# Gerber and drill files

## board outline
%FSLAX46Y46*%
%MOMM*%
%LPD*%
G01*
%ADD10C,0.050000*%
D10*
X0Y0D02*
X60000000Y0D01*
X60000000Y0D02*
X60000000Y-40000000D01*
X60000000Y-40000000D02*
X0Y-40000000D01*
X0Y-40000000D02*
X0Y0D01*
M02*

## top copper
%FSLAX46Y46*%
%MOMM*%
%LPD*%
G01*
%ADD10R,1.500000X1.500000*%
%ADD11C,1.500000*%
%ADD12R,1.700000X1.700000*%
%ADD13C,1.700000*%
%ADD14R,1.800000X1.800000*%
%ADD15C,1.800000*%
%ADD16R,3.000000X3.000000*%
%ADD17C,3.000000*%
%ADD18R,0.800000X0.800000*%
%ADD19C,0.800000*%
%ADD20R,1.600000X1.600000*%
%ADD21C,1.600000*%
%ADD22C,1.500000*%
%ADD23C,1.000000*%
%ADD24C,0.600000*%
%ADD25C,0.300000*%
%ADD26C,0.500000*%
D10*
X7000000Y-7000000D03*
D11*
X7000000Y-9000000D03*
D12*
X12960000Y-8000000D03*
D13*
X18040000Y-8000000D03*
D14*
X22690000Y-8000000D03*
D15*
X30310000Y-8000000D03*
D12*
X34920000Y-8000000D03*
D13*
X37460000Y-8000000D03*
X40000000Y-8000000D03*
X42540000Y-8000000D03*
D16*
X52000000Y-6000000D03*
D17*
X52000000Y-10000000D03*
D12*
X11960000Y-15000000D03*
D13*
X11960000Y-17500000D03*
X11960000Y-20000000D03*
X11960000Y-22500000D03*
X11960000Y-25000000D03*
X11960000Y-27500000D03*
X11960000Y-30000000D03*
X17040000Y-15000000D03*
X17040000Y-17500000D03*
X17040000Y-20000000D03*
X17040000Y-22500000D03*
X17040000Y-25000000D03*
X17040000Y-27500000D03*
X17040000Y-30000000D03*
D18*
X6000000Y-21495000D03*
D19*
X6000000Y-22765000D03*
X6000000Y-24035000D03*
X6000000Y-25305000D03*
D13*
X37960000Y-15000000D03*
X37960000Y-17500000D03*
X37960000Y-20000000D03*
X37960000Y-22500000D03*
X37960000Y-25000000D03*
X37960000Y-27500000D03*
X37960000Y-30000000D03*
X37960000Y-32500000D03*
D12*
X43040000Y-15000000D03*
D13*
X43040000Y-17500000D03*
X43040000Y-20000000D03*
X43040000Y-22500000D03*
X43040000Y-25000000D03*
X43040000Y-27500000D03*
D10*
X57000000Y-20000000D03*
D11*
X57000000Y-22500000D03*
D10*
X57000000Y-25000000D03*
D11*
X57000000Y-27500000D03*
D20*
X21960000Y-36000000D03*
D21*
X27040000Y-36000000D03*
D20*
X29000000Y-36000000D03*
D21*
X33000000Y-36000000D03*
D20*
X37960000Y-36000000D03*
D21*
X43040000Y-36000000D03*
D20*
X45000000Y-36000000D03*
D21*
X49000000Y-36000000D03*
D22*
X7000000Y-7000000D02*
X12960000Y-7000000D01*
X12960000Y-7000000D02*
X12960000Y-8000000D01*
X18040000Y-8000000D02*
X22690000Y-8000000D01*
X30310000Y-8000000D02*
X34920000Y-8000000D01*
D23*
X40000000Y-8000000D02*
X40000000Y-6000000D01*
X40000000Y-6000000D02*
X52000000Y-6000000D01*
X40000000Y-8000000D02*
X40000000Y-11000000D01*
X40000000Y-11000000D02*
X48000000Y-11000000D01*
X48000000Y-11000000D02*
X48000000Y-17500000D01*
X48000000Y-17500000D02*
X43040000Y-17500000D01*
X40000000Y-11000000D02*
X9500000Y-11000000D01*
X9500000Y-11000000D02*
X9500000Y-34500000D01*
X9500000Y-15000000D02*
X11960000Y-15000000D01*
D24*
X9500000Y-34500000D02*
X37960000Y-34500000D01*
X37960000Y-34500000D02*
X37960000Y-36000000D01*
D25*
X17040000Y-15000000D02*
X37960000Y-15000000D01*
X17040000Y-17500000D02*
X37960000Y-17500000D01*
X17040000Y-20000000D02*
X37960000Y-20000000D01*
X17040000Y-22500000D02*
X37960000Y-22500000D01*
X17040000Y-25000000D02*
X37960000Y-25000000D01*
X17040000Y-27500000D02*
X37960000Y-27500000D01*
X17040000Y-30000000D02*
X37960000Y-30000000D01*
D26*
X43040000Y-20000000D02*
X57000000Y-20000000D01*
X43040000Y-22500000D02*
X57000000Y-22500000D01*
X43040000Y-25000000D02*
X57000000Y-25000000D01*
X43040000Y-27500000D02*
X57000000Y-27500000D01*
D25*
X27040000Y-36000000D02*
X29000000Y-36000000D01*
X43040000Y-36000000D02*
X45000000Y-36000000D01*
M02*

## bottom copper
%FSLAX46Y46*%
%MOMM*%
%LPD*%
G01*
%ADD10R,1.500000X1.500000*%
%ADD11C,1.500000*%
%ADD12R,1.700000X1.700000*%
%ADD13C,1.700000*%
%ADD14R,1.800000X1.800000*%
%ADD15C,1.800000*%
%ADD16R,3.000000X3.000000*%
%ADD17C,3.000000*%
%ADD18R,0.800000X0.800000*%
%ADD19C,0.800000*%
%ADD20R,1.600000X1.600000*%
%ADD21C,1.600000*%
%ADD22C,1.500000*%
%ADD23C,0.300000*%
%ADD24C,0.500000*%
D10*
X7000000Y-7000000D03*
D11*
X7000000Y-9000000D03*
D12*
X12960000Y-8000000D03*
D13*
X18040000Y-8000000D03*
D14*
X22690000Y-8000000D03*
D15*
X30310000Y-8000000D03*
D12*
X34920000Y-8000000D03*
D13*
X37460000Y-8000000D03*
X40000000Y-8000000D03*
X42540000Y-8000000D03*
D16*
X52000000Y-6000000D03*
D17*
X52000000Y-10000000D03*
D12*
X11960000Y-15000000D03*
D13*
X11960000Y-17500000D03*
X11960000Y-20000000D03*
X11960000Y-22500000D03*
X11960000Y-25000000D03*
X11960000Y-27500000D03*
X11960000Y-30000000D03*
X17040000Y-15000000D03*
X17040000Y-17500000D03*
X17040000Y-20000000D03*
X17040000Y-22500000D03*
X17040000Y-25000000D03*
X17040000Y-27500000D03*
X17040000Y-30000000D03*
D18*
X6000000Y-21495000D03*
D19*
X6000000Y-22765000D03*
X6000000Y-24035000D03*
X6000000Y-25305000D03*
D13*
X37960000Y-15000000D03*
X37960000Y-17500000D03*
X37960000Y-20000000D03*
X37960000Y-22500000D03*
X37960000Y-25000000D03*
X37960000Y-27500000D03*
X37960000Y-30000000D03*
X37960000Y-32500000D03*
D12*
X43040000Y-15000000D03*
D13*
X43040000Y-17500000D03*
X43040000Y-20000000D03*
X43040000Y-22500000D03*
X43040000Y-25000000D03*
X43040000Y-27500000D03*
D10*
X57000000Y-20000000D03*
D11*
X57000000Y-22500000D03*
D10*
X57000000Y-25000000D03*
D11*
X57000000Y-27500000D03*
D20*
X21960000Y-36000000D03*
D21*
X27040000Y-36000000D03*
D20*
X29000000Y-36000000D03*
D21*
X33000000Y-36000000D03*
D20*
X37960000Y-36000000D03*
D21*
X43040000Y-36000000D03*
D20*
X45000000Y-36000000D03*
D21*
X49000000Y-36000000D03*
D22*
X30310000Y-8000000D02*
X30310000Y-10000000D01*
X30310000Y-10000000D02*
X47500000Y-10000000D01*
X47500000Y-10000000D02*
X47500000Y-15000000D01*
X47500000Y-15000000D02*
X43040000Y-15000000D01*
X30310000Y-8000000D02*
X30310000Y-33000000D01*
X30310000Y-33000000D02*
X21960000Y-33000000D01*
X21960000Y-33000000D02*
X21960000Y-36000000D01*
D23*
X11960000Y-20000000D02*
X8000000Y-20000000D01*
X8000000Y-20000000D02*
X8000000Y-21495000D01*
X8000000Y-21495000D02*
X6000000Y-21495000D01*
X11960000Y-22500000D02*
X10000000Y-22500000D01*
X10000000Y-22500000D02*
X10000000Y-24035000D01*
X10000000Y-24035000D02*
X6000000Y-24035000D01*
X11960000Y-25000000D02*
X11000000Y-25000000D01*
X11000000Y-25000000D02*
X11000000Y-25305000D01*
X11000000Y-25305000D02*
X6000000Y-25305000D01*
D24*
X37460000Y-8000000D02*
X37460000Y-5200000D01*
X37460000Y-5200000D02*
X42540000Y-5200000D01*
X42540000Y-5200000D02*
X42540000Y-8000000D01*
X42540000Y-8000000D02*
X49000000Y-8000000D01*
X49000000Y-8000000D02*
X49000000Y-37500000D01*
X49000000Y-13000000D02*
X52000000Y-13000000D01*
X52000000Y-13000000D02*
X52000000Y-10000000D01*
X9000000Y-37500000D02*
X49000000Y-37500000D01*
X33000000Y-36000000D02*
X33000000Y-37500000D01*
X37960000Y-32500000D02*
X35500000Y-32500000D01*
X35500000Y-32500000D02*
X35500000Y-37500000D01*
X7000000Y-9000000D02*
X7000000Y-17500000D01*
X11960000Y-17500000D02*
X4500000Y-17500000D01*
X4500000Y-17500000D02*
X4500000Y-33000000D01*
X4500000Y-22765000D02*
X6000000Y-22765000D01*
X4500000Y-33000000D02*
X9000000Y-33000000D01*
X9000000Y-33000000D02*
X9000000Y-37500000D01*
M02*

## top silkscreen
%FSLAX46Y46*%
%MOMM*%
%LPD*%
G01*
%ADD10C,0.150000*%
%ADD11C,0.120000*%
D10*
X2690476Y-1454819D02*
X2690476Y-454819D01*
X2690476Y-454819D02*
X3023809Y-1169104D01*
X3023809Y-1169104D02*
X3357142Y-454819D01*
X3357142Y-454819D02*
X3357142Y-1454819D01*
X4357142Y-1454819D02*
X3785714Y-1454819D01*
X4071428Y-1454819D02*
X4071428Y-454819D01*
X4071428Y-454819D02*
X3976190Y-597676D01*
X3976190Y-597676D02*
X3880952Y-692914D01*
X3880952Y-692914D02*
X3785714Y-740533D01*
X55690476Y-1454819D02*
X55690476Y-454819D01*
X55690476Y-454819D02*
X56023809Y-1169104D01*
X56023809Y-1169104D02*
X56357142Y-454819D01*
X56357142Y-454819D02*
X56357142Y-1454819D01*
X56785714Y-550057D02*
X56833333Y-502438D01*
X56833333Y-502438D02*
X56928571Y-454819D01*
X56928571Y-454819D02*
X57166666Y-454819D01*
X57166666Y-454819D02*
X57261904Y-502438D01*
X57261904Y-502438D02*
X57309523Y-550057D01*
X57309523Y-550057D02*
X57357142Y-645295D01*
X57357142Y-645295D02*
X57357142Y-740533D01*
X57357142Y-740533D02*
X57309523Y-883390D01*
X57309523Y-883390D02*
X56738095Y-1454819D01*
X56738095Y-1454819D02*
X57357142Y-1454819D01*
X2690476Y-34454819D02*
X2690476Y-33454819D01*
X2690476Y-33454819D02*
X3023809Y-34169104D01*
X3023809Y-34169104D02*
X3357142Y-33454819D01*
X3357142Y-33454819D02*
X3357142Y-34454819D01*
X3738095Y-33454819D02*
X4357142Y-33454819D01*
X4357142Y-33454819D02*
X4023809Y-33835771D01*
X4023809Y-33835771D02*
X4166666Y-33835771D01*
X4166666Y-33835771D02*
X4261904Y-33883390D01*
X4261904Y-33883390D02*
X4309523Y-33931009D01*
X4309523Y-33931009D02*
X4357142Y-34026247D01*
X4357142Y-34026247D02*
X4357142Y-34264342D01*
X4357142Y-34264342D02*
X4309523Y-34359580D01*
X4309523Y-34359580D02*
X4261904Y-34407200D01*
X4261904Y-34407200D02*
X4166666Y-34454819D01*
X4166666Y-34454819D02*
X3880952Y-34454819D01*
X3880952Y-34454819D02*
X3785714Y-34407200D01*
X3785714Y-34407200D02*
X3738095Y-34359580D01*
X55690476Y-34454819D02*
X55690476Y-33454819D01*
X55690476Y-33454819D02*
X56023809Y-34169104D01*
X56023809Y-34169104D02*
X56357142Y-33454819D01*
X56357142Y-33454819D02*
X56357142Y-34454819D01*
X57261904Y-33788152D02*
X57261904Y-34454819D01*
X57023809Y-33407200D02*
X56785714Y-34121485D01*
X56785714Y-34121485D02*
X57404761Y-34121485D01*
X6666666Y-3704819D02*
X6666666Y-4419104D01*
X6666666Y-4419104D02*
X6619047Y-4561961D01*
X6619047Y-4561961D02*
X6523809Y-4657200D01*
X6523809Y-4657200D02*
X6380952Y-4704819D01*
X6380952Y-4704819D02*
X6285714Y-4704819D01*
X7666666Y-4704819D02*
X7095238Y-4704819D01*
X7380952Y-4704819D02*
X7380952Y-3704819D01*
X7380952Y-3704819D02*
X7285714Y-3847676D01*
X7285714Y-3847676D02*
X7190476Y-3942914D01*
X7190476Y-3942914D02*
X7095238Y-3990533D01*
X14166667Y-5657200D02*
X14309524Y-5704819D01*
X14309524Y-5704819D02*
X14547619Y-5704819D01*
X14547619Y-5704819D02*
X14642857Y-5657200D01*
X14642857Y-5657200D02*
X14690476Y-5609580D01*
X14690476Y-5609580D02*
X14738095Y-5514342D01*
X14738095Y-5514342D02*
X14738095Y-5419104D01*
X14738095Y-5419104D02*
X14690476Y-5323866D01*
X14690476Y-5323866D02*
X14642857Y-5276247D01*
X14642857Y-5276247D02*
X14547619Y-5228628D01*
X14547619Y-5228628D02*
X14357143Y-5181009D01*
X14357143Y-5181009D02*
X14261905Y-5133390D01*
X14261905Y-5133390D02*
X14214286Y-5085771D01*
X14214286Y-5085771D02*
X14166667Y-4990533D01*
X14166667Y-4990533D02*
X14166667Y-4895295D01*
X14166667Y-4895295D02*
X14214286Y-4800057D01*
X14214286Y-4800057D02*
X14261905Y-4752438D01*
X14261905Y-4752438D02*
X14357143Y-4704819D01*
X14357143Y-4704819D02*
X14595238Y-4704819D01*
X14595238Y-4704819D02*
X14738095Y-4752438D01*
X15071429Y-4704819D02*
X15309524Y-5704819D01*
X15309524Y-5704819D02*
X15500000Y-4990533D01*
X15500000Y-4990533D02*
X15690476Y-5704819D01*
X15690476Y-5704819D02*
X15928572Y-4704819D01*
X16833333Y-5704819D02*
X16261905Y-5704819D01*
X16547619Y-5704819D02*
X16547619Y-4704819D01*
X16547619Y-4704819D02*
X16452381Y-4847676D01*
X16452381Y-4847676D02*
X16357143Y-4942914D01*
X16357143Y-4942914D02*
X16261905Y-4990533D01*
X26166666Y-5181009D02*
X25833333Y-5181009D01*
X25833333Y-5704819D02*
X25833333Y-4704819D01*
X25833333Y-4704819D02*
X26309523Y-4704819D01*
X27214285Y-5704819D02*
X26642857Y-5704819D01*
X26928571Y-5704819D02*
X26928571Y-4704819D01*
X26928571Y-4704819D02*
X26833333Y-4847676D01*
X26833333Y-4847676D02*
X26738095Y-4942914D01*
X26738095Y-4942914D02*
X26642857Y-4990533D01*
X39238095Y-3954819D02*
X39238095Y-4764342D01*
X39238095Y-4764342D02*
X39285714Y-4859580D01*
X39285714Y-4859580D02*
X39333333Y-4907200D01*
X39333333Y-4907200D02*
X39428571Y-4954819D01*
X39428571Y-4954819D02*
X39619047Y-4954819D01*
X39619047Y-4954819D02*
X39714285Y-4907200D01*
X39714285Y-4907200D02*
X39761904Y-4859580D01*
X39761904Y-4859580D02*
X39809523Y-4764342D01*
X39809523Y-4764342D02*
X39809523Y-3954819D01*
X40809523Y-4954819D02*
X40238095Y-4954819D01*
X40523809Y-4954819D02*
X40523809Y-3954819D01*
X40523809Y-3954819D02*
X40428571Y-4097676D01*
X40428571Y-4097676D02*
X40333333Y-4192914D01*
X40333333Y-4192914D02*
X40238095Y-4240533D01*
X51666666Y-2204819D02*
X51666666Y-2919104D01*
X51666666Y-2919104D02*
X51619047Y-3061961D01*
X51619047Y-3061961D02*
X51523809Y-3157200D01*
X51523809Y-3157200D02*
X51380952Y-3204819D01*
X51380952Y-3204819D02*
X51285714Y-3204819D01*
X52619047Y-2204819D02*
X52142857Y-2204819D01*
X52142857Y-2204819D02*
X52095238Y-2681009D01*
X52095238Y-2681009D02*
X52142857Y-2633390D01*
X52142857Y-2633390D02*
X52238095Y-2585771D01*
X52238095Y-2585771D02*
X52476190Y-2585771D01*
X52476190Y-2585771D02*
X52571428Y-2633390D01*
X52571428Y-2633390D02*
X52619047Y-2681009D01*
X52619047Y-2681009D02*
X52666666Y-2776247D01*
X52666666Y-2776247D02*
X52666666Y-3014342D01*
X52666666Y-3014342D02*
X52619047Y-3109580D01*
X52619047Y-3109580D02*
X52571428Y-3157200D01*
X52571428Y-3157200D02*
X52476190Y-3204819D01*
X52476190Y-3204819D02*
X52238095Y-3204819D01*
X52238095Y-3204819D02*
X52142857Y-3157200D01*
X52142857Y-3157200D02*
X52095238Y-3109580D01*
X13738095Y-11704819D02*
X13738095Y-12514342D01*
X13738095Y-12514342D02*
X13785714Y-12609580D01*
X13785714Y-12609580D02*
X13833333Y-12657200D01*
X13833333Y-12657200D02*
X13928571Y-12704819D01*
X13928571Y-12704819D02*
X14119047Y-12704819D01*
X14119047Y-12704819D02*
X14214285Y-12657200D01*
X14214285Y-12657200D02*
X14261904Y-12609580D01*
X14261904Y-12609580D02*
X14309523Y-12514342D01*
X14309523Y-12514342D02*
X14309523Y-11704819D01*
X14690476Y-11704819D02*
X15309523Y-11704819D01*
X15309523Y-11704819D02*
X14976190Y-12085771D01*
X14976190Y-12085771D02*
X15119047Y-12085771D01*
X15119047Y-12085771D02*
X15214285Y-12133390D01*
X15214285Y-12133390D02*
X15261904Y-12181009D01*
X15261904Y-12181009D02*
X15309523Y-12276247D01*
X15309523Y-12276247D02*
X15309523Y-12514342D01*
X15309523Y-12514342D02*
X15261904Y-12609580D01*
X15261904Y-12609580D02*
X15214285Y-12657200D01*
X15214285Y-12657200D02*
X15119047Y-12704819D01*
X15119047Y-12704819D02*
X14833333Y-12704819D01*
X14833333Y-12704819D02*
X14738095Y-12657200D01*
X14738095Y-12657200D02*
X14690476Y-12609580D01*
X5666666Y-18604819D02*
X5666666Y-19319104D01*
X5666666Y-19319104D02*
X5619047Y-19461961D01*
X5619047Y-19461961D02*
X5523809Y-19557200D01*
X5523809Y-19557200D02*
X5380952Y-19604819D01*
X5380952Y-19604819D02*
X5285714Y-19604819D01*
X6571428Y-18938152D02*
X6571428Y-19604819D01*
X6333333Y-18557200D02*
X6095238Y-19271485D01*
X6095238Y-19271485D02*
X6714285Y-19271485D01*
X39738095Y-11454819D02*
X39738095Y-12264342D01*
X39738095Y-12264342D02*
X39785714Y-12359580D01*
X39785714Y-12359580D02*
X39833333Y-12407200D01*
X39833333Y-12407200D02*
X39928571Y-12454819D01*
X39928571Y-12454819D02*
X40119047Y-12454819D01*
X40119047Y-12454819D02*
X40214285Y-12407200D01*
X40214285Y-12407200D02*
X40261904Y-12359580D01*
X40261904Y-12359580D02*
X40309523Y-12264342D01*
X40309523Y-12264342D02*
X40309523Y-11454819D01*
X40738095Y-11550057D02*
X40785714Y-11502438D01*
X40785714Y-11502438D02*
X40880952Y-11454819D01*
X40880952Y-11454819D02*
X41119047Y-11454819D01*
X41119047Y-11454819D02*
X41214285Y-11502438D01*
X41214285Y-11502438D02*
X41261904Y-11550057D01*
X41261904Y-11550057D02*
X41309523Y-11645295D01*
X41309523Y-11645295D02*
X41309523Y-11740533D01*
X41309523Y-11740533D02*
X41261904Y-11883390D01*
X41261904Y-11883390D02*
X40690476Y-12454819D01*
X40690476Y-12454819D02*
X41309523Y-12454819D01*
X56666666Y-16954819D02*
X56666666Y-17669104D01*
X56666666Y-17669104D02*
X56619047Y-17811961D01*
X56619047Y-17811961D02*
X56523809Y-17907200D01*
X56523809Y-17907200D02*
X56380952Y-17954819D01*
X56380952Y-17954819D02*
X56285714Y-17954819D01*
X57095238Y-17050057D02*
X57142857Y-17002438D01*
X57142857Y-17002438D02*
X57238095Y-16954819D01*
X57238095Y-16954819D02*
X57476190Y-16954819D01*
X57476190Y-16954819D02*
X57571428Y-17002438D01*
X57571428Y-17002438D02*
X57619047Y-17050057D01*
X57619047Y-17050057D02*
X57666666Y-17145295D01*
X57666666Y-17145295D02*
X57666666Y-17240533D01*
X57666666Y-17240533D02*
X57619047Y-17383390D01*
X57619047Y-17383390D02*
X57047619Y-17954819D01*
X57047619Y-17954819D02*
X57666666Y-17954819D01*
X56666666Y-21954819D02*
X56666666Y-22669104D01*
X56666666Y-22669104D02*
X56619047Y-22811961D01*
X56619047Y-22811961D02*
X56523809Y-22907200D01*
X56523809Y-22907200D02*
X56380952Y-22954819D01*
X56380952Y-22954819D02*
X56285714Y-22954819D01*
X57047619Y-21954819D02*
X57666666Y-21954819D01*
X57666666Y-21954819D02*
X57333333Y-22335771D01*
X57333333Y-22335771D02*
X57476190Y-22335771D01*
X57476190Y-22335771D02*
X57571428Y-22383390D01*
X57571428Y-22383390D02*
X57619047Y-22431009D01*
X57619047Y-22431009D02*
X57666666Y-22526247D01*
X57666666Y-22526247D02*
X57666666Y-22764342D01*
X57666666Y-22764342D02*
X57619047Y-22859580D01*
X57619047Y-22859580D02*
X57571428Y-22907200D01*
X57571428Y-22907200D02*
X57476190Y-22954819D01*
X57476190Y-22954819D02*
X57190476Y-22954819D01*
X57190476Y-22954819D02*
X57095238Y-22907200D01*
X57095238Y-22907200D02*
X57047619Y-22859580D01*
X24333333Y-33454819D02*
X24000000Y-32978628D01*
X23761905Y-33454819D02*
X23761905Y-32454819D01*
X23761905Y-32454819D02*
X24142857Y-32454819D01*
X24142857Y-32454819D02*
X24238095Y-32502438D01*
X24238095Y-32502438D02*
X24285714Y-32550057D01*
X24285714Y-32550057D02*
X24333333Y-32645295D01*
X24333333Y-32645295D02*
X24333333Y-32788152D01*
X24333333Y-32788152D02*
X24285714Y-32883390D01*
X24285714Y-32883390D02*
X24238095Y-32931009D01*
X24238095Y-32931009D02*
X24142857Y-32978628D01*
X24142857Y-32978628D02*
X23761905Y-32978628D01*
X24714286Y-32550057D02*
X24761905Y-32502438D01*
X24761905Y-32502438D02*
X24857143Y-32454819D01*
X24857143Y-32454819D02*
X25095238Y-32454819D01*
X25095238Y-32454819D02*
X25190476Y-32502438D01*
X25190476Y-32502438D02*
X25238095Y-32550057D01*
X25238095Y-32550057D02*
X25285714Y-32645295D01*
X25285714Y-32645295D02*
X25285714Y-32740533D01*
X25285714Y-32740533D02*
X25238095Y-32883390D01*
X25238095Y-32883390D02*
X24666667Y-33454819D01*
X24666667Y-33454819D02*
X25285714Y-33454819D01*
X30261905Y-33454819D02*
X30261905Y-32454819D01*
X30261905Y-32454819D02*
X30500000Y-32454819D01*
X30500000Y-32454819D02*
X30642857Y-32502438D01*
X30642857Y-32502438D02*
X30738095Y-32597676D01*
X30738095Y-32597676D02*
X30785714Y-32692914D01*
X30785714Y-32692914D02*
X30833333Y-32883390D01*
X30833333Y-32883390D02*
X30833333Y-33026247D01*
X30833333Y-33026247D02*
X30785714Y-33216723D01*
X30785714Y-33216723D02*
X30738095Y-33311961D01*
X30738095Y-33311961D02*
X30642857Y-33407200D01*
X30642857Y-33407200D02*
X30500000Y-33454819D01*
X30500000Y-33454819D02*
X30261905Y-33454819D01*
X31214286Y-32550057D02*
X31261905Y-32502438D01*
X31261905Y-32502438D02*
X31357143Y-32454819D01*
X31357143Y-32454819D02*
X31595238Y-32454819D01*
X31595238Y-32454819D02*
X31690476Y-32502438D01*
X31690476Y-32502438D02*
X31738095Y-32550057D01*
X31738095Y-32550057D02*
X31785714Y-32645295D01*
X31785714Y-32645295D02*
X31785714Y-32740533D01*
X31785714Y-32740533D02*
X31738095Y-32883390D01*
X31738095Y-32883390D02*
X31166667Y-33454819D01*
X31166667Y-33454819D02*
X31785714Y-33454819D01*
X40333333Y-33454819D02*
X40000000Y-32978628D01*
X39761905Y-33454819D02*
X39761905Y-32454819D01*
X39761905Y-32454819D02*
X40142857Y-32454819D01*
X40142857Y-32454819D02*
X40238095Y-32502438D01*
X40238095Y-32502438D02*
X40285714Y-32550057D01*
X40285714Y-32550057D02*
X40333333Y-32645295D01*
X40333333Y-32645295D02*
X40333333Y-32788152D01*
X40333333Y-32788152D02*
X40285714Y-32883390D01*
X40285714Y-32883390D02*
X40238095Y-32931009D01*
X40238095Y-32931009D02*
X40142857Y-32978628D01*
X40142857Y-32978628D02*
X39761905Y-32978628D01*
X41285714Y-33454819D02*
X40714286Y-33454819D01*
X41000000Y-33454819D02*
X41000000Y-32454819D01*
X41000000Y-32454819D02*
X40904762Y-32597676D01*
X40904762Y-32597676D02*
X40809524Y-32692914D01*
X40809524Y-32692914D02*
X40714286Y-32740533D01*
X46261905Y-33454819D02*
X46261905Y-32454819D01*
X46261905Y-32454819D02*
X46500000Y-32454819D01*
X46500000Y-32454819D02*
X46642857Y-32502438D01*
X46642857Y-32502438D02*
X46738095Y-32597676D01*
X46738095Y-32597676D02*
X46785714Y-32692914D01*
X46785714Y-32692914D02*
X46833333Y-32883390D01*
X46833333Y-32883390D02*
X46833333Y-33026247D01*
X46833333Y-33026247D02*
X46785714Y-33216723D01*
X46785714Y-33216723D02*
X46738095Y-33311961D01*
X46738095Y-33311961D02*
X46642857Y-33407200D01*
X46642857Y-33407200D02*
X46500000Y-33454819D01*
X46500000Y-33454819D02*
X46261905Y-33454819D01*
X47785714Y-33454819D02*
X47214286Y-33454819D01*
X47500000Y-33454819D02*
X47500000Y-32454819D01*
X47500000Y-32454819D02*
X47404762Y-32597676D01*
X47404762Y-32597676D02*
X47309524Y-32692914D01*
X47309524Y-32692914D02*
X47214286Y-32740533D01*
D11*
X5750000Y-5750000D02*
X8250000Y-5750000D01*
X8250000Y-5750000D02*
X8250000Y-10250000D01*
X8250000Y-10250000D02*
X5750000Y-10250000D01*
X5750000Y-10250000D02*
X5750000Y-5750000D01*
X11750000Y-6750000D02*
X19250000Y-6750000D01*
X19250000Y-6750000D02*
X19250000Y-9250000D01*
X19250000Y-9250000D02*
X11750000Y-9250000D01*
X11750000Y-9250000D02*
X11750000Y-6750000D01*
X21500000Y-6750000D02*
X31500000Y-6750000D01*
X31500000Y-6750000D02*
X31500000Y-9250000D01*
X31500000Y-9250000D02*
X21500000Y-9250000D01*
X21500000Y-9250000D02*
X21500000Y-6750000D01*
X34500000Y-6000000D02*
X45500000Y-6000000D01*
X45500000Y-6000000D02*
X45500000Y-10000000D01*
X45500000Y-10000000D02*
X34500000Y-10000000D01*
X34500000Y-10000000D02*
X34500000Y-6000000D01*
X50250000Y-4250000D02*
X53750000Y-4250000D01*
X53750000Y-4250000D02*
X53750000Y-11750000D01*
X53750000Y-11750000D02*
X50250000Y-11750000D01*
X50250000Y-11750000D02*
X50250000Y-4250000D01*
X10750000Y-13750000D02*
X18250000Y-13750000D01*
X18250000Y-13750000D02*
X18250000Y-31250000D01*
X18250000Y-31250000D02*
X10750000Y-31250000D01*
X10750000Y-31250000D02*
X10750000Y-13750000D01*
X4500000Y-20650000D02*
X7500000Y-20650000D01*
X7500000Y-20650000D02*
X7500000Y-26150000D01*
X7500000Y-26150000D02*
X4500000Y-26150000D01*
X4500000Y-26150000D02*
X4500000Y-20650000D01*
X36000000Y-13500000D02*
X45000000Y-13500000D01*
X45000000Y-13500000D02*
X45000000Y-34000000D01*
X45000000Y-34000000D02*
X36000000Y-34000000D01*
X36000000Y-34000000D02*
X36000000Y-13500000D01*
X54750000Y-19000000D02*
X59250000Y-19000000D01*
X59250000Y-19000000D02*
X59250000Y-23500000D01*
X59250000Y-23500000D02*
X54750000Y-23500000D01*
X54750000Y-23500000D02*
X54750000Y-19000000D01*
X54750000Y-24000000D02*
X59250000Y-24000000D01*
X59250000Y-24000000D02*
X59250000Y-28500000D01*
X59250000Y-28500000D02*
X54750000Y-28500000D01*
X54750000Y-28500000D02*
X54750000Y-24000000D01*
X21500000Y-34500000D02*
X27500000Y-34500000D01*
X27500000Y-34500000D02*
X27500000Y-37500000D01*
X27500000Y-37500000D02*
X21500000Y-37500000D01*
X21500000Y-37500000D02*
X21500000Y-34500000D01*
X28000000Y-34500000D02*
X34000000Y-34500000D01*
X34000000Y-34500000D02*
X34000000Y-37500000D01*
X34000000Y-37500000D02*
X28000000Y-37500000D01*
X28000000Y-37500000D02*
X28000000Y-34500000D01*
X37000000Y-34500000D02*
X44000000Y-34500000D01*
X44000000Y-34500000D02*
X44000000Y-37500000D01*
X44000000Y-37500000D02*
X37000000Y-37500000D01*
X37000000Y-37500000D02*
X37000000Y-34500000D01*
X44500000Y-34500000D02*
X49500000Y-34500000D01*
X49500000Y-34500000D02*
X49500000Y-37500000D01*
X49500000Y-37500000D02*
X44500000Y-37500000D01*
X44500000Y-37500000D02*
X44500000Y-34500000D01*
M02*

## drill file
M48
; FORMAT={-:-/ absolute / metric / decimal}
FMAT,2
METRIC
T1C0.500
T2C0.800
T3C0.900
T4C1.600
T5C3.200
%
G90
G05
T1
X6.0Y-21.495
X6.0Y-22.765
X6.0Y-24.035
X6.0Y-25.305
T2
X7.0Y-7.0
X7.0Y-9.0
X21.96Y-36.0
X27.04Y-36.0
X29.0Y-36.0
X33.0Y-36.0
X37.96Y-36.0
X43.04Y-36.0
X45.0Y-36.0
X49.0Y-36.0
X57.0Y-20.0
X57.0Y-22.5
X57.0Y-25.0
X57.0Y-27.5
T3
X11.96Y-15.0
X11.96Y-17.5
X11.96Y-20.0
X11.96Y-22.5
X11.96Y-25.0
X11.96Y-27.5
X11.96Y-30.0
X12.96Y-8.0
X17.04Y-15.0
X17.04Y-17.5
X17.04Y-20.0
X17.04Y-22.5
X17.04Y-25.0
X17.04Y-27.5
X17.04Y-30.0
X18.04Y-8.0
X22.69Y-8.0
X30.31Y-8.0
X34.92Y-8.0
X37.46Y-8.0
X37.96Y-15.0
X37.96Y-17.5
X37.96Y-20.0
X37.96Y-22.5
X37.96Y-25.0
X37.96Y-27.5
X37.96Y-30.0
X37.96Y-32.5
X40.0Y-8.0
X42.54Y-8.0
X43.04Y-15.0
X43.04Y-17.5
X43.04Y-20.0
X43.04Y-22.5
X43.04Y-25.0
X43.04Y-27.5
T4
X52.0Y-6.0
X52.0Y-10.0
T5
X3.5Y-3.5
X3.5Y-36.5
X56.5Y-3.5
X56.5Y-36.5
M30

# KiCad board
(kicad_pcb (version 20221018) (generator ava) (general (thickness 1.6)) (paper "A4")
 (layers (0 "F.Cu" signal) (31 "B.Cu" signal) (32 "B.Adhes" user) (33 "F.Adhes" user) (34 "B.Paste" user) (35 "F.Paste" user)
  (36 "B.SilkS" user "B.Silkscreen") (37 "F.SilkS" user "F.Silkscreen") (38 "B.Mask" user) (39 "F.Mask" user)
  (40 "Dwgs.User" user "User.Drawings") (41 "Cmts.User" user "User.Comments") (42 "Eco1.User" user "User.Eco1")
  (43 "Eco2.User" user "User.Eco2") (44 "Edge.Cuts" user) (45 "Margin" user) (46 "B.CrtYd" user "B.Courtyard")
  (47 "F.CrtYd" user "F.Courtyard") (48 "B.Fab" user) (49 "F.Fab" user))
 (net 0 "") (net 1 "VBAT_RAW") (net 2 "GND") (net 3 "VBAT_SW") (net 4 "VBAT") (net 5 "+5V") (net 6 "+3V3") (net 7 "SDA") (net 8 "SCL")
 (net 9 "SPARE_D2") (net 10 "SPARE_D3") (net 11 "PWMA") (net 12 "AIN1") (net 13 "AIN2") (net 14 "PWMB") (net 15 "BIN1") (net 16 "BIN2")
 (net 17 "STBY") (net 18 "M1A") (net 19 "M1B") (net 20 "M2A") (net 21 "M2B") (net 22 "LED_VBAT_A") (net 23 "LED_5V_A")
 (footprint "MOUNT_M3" (layer "F.Cu") (at 3.5 3.5)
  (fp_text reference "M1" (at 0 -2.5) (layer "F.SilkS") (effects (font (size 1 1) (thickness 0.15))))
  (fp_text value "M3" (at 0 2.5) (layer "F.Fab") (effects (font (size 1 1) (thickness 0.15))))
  (pad "" np_thru_hole circle (at 0 0) (size 3.2 3.2) (drill 3.2) (layers "*.Cu" "*.Mask")))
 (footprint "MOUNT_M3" (layer "F.Cu") (at 56.5 3.5)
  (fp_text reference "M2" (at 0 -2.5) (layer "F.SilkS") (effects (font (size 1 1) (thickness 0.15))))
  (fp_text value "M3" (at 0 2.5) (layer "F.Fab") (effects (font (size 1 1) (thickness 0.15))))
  (pad "" np_thru_hole circle (at 0 0) (size 3.2 3.2) (drill 3.2) (layers "*.Cu" "*.Mask")))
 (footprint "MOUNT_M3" (layer "F.Cu") (at 3.5 36.5)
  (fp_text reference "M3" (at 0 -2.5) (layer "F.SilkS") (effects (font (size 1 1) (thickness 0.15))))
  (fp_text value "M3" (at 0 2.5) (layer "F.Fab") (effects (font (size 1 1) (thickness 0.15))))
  (pad "" np_thru_hole circle (at 0 0) (size 3.2 3.2) (drill 3.2) (layers "*.Cu" "*.Mask")))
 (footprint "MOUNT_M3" (layer "F.Cu") (at 56.5 36.5)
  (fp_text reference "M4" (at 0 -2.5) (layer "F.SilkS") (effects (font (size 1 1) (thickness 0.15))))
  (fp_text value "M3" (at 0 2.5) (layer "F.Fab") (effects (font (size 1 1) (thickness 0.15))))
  (pad "" np_thru_hole circle (at 0 0) (size 3.2 3.2) (drill 3.2) (layers "*.Cu" "*.Mask")))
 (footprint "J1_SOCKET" (layer "F.Cu") (at 7 8)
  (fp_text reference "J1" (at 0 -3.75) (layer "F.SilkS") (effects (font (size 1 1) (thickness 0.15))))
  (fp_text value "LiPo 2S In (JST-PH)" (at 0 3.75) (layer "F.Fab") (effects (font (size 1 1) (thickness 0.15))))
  (fp_line (start -1.25 -2.25) (end 1.25 -2.25) (layer "F.SilkS") (width 0.12))
  (fp_line (start 1.25 -2.25) (end 1.25 2.25) (layer "F.SilkS") (width 0.12))
  (fp_line (start 1.25 2.25) (end -1.25 2.25) (layer "F.SilkS") (width 0.12))
  (fp_line (start -1.25 2.25) (end -1.25 -2.25) (layer "F.SilkS") (width 0.12))
  (pad "1" thru_hole rect (at 0 -1) (size 1.5 1.5) (drill 0.8) (layers "*.Cu" "*.Mask") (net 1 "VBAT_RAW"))
  (pad "2" thru_hole circle (at 0 1) (size 1.5 1.5) (drill 0.8) (layers "*.Cu" "*.Mask") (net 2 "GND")))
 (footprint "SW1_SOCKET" (layer "F.Cu") (at 15.5 8)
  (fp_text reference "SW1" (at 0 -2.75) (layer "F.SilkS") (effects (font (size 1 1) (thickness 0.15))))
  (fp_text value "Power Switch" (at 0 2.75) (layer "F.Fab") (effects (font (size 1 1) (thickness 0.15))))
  (fp_line (start -3.75 -1.25) (end 3.75 -1.25) (layer "F.SilkS") (width 0.12))
  (fp_line (start 3.75 -1.25) (end 3.75 1.25) (layer "F.SilkS") (width 0.12))
  (fp_line (start 3.75 1.25) (end -3.75 1.25) (layer "F.SilkS") (width 0.12))
  (fp_line (start -3.75 1.25) (end -3.75 -1.25) (layer "F.SilkS") (width 0.12))
  (pad "1" thru_hole rect (at -2.54 0) (size 1.7 1.7) (drill 0.9) (layers "*.Cu" "*.Mask") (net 1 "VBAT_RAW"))
  (pad "2" thru_hole circle (at 2.54 0) (size 1.7 1.7) (drill 0.9) (layers "*.Cu" "*.Mask") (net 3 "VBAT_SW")))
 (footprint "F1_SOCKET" (layer "F.Cu") (at 26.5 8)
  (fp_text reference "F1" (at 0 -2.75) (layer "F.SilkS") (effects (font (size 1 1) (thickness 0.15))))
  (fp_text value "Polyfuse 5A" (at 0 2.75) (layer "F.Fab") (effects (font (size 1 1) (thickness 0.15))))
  (fp_line (start -5.0 -1.25) (end 5.0 -1.25) (layer "F.SilkS") (width 0.12))
  (fp_line (start 5.0 -1.25) (end 5.0 1.25) (layer "F.SilkS") (width 0.12))
  (fp_line (start 5.0 1.25) (end -5.0 1.25) (layer "F.SilkS") (width 0.12))
  (fp_line (start -5.0 1.25) (end -5.0 -1.25) (layer "F.SilkS") (width 0.12))
  (pad "1" thru_hole rect (at -3.81 0) (size 1.8 1.8) (drill 0.9) (layers "*.Cu" "*.Mask") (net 3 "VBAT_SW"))
  (pad "2" thru_hole circle (at 3.81 0) (size 1.8 1.8) (drill 0.9) (layers "*.Cu" "*.Mask") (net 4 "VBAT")))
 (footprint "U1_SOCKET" (layer "F.Cu") (at 40 8)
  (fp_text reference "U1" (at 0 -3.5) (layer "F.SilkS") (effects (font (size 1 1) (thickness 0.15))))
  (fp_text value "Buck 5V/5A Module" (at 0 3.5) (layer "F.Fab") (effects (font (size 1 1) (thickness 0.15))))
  (fp_line (start -5.5 -2.0) (end 5.5 -2.0) (layer "F.SilkS") (width 0.12))
  (fp_line (start 5.5 -2.0) (end 5.5 2.0) (layer "F.SilkS") (width 0.12))
  (fp_line (start 5.5 2.0) (end -5.5 2.0) (layer "F.SilkS") (width 0.12))
  (fp_line (start -5.5 2.0) (end -5.5 -2.0) (layer "F.SilkS") (width 0.12))
  (pad "1" thru_hole rect (at -5.08 0) (size 1.7 1.7) (drill 0.9) (layers "*.Cu" "*.Mask") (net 4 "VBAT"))
  (pad "2" thru_hole circle (at -2.54 0) (size 1.7 1.7) (drill 0.9) (layers "*.Cu" "*.Mask") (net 2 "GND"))
  (pad "3" thru_hole circle (at 0 0) (size 1.7 1.7) (drill 0.9) (layers "*.Cu" "*.Mask") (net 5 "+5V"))
  (pad "4" thru_hole circle (at 2.54 0) (size 1.7 1.7) (drill 0.9) (layers "*.Cu" "*.Mask") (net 2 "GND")))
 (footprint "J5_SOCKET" (layer "F.Cu") (at 52 8)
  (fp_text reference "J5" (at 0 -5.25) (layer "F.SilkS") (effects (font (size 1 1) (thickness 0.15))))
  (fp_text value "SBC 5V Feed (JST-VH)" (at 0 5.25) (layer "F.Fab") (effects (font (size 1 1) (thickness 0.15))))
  (fp_line (start -1.75 -3.75) (end 1.75 -3.75) (layer "F.SilkS") (width 0.12))
  (fp_line (start 1.75 -3.75) (end 1.75 3.75) (layer "F.SilkS") (width 0.12))
  (fp_line (start 1.75 3.75) (end -1.75 3.75) (layer "F.SilkS") (width 0.12))
  (fp_line (start -1.75 3.75) (end -1.75 -3.75) (layer "F.SilkS") (width 0.12))
  (pad "1" thru_hole rect (at 0 -2) (size 3.0 3.0) (drill 1.6) (layers "*.Cu" "*.Mask") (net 5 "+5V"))
  (pad "2" thru_hole circle (at 0 2) (size 3.0 3.0) (drill 1.6) (layers "*.Cu" "*.Mask") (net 2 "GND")))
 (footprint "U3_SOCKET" (layer "F.Cu") (at 14.5 22.5)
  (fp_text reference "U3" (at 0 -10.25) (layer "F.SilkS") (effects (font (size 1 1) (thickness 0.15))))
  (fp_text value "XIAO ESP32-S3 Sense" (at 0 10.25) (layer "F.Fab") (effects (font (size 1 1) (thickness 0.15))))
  (fp_line (start -3.75 -8.75) (end 3.75 -8.75) (layer "F.SilkS") (width 0.12))
  (fp_line (start 3.75 -8.75) (end 3.75 8.75) (layer "F.SilkS") (width 0.12))
  (fp_line (start 3.75 8.75) (end -3.75 8.75) (layer "F.SilkS") (width 0.12))
  (fp_line (start -3.75 8.75) (end -3.75 -8.75) (layer "F.SilkS") (width 0.12))
  (pad "1" thru_hole rect (at -2.54 -7.5) (size 1.7 1.7) (drill 0.9) (layers "*.Cu" "*.Mask") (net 5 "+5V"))
  (pad "2" thru_hole circle (at -2.54 -5.0) (size 1.7 1.7) (drill 0.9) (layers "*.Cu" "*.Mask") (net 2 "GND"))
  (pad "3" thru_hole circle (at -2.54 -2.5) (size 1.7 1.7) (drill 0.9) (layers "*.Cu" "*.Mask") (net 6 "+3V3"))
  (pad "4" thru_hole circle (at -2.54 0.0) (size 1.7 1.7) (drill 0.9) (layers "*.Cu" "*.Mask") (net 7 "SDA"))
  (pad "5" thru_hole circle (at -2.54 2.5) (size 1.7 1.7) (drill 0.9) (layers "*.Cu" "*.Mask") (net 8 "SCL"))
  (pad "6" thru_hole circle (at -2.54 5.0) (size 1.7 1.7) (drill 0.9) (layers "*.Cu" "*.Mask") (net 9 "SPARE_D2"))
  (pad "7" thru_hole circle (at -2.54 7.5) (size 1.7 1.7) (drill 0.9) (layers "*.Cu" "*.Mask") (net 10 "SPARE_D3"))
  (pad "8" thru_hole circle (at 2.54 -7.5) (size 1.7 1.7) (drill 0.9) (layers "*.Cu" "*.Mask") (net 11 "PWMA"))
  (pad "9" thru_hole circle (at 2.54 -5.0) (size 1.7 1.7) (drill 0.9) (layers "*.Cu" "*.Mask") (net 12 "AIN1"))
  (pad "10" thru_hole circle (at 2.54 -2.5) (size 1.7 1.7) (drill 0.9) (layers "*.Cu" "*.Mask") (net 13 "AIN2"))
  (pad "11" thru_hole circle (at 2.54 0.0) (size 1.7 1.7) (drill 0.9) (layers "*.Cu" "*.Mask") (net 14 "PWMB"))
  (pad "12" thru_hole circle (at 2.54 2.5) (size 1.7 1.7) (drill 0.9) (layers "*.Cu" "*.Mask") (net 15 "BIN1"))
  (pad "13" thru_hole circle (at 2.54 5.0) (size 1.7 1.7) (drill 0.9) (layers "*.Cu" "*.Mask") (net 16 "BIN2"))
  (pad "14" thru_hole circle (at 2.54 7.5) (size 1.7 1.7) (drill 0.9) (layers "*.Cu" "*.Mask") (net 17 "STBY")))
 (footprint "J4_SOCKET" (layer "F.Cu") (at 6 23.4)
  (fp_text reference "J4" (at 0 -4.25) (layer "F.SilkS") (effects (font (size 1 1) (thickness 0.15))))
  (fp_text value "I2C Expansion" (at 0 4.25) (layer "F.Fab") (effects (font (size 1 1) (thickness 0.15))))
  (fp_line (start -1.5 -2.75) (end 1.5 -2.75) (layer "F.SilkS") (width 0.12))
  (fp_line (start 1.5 -2.75) (end 1.5 2.75) (layer "F.SilkS") (width 0.12))
  (fp_line (start 1.5 2.75) (end -1.5 2.75) (layer "F.SilkS") (width 0.12))
  (fp_line (start -1.5 2.75) (end -1.5 -2.75) (layer "F.SilkS") (width 0.12))
  (pad "1" thru_hole rect (at 0 -1.905) (size 0.8 0.8) (drill 0.5) (layers "*.Cu" "*.Mask") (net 6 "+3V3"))
  (pad "2" thru_hole circle (at 0 -0.635) (size 0.8 0.8) (drill 0.5) (layers "*.Cu" "*.Mask") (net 2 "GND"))
  (pad "3" thru_hole circle (at 0 0.635) (size 0.8 0.8) (drill 0.5) (layers "*.Cu" "*.Mask") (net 7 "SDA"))
  (pad "4" thru_hole circle (at 0 1.905) (size 0.8 0.8) (drill 0.5) (layers "*.Cu" "*.Mask") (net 8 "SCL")))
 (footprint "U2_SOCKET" (layer "F.Cu") (at 40.5 23.75)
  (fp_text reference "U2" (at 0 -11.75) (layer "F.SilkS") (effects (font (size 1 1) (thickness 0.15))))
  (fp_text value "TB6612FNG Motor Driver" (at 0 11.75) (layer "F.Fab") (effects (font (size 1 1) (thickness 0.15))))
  (fp_line (start -4.5 -10.25) (end 4.5 -10.25) (layer "F.SilkS") (width 0.12))
  (fp_line (start 4.5 -10.25) (end 4.5 10.25) (layer "F.SilkS") (width 0.12))
  (fp_line (start 4.5 10.25) (end -4.5 10.25) (layer "F.SilkS") (width 0.12))
  (fp_line (start -4.5 10.25) (end -4.5 -10.25) (layer "F.SilkS") (width 0.12))
  (pad "4" thru_hole circle (at -2.54 -8.75) (size 1.7 1.7) (drill 0.9) (layers "*.Cu" "*.Mask") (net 11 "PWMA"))
  (pad "5" thru_hole circle (at -2.54 -6.25) (size 1.7 1.7) (drill 0.9) (layers "*.Cu" "*.Mask") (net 12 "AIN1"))
  (pad "6" thru_hole circle (at -2.54 -3.75) (size 1.7 1.7) (drill 0.9) (layers "*.Cu" "*.Mask") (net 13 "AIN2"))
  (pad "7" thru_hole circle (at -2.54 -1.25) (size 1.7 1.7) (drill 0.9) (layers "*.Cu" "*.Mask") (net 14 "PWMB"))
  (pad "8" thru_hole circle (at -2.54 1.25) (size 1.7 1.7) (drill 0.9) (layers "*.Cu" "*.Mask") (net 15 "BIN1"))
  (pad "9" thru_hole circle (at -2.54 3.75) (size 1.7 1.7) (drill 0.9) (layers "*.Cu" "*.Mask") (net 16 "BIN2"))
  (pad "10" thru_hole circle (at -2.54 6.25) (size 1.7 1.7) (drill 0.9) (layers "*.Cu" "*.Mask") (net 17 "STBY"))
  (pad "3" thru_hole circle (at -2.54 8.75) (size 1.7 1.7) (drill 0.9) (layers "*.Cu" "*.Mask") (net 2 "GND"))
  (pad "1" thru_hole rect (at 2.54 -8.75) (size 1.7 1.7) (drill 0.9) (layers "*.Cu" "*.Mask") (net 4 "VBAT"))
  (pad "2" thru_hole circle (at 2.54 -6.25) (size 1.7 1.7) (drill 0.9) (layers "*.Cu" "*.Mask") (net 5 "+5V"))
  (pad "11" thru_hole circle (at 2.54 -3.75) (size 1.7 1.7) (drill 0.9) (layers "*.Cu" "*.Mask") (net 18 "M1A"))
  (pad "12" thru_hole circle (at 2.54 -1.25) (size 1.7 1.7) (drill 0.9) (layers "*.Cu" "*.Mask") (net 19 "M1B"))
  (pad "13" thru_hole circle (at 2.54 1.25) (size 1.7 1.7) (drill 0.9) (layers "*.Cu" "*.Mask") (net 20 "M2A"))
  (pad "14" thru_hole circle (at 2.54 3.75) (size 1.7 1.7) (drill 0.9) (layers "*.Cu" "*.Mask") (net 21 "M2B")))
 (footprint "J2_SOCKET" (layer "F.Cu") (at 57 21.25)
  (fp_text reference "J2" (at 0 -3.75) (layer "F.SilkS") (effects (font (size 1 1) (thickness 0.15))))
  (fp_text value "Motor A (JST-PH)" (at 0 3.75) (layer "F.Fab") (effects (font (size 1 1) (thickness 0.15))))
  (fp_line (start -2.25 -2.25) (end 2.25 -2.25) (layer "F.SilkS") (width 0.12))
  (fp_line (start 2.25 -2.25) (end 2.25 2.25) (layer "F.SilkS") (width 0.12))
  (fp_line (start 2.25 2.25) (end -2.25 2.25) (layer "F.SilkS") (width 0.12))
  (fp_line (start -2.25 2.25) (end -2.25 -2.25) (layer "F.SilkS") (width 0.12))
  (pad "1" thru_hole rect (at 0 -1.25) (size 1.5 1.5) (drill 0.8) (layers "*.Cu" "*.Mask") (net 18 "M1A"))
  (pad "2" thru_hole circle (at 0 1.25) (size 1.5 1.5) (drill 0.8) (layers "*.Cu" "*.Mask") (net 19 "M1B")))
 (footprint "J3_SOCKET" (layer "F.Cu") (at 57 26.25)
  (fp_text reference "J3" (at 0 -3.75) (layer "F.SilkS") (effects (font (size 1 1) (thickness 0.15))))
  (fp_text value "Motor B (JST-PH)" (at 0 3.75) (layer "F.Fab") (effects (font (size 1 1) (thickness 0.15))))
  (fp_line (start -2.25 -2.25) (end 2.25 -2.25) (layer "F.SilkS") (width 0.12))
  (fp_line (start 2.25 -2.25) (end 2.25 2.25) (layer "F.SilkS") (width 0.12))
  (fp_line (start 2.25 2.25) (end -2.25 2.25) (layer "F.SilkS") (width 0.12))
  (fp_line (start -2.25 2.25) (end -2.25 -2.25) (layer "F.SilkS") (width 0.12))
  (pad "1" thru_hole rect (at 0 -1.25) (size 1.5 1.5) (drill 0.8) (layers "*.Cu" "*.Mask") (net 20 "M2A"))
  (pad "2" thru_hole circle (at 0 1.25) (size 1.5 1.5) (drill 0.8) (layers "*.Cu" "*.Mask") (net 21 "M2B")))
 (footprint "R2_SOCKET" (layer "F.Cu") (at 24.5 36)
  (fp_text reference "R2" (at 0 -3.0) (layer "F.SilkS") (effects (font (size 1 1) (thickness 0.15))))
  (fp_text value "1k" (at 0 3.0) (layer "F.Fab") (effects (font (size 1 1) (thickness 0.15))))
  (fp_line (start -3.0 -1.5) (end 3.0 -1.5) (layer "F.SilkS") (width 0.12))
  (fp_line (start 3.0 -1.5) (end 3.0 1.5) (layer "F.SilkS") (width 0.12))
  (fp_line (start 3.0 1.5) (end -3.0 1.5) (layer "F.SilkS") (width 0.12))
  (fp_line (start -3.0 1.5) (end -3.0 -1.5) (layer "F.SilkS") (width 0.12))
  (pad "1" thru_hole rect (at -2.54 0) (size 1.6 1.6) (drill 0.8) (layers "*.Cu" "*.Mask") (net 4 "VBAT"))
  (pad "2" thru_hole circle (at 2.54 0) (size 1.6 1.6) (drill 0.8) (layers "*.Cu" "*.Mask") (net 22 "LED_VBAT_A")))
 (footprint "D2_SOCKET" (layer "F.Cu") (at 31 36)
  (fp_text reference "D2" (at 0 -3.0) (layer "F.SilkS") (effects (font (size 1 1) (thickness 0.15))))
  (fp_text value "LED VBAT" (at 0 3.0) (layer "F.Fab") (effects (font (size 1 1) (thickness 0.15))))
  (fp_line (start -3.0 -1.5) (end 3.0 -1.5) (layer "F.SilkS") (width 0.12))
  (fp_line (start 3.0 -1.5) (end 3.0 1.5) (layer "F.SilkS") (width 0.12))
  (fp_line (start 3.0 1.5) (end -3.0 1.5) (layer "F.SilkS") (width 0.12))
  (fp_line (start -3.0 1.5) (end -3.0 -1.5) (layer "F.SilkS") (width 0.12))
  (pad "1" thru_hole rect (at -2 0) (size 1.6 1.6) (drill 0.8) (layers "*.Cu" "*.Mask") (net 22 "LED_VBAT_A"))
  (pad "2" thru_hole circle (at 2 0) (size 1.6 1.6) (drill 0.8) (layers "*.Cu" "*.Mask") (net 2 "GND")))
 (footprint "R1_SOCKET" (layer "F.Cu") (at 40.5 36)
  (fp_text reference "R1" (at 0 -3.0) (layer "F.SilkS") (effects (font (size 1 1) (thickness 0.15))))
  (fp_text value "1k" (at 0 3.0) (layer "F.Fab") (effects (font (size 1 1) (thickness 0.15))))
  (fp_line (start -3.5 -1.5) (end 3.5 -1.5) (layer "F.SilkS") (width 0.12))
  (fp_line (start 3.5 -1.5) (end 3.5 1.5) (layer "F.SilkS") (width 0.12))
  (fp_line (start 3.5 1.5) (end -3.5 1.5) (layer "F.SilkS") (width 0.12))
  (fp_line (start -3.5 1.5) (end -3.5 -1.5) (layer "F.SilkS") (width 0.12))
  (pad "1" thru_hole rect (at -2.54 0) (size 1.6 1.6) (drill 0.8) (layers "*.Cu" "*.Mask") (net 5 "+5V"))
  (pad "2" thru_hole circle (at 2.54 0) (size 1.6 1.6) (drill 0.8) (layers "*.Cu" "*.Mask") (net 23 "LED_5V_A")))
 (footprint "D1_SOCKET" (layer "F.Cu") (at 47 36)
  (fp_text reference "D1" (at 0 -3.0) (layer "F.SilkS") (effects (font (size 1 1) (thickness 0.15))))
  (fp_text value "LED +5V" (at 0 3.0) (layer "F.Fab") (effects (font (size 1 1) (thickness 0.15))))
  (fp_line (start -2.5 -1.5) (end 2.5 -1.5) (layer "F.SilkS") (width 0.12))
  (fp_line (start 2.5 -1.5) (end 2.5 1.5) (layer "F.SilkS") (width 0.12))
  (fp_line (start 2.5 1.5) (end -2.5 1.5) (layer "F.SilkS") (width 0.12))
  (fp_line (start -2.5 1.5) (end -2.5 -1.5) (layer "F.SilkS") (width 0.12))
  (pad "1" thru_hole rect (at -2 0) (size 1.6 1.6) (drill 0.8) (layers "*.Cu" "*.Mask") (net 23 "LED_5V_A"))
  (pad "2" thru_hole circle (at 2 0) (size 1.6 1.6) (drill 0.8) (layers "*.Cu" "*.Mask") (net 2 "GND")))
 (segment (start 7 7) (end 12.96 7) (width 1.5) (layer "F.Cu") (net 1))
 (segment (start 12.96 7) (end 12.96 8) (width 1.5) (layer "F.Cu") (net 1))
 (segment (start 18.04 8) (end 22.69 8) (width 1.5) (layer "F.Cu") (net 3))
 (segment (start 30.31 8) (end 34.92 8) (width 1.5) (layer "F.Cu") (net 4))
 (segment (start 30.31 8) (end 30.31 10) (width 1.5) (layer "B.Cu") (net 4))
 (segment (start 30.31 10) (end 47.5 10.0) (width 1.5) (layer "B.Cu") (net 4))
 (segment (start 47.5 10.0) (end 47.5 15.0) (width 1.5) (layer "B.Cu") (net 4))
 (segment (start 47.5 15.0) (end 43.04 15.0) (width 1.5) (layer "B.Cu") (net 4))
 (segment (start 30.31 8) (end 30.31 33) (width 1.5) (layer "B.Cu") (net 4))
 (segment (start 30.31 33) (end 21.96 33) (width 1.5) (layer "B.Cu") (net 4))
 (segment (start 21.96 33) (end 21.96 36) (width 1.5) (layer "B.Cu") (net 4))
 (segment (start 40 8) (end 40 6) (width 1.0) (layer "F.Cu") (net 5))
 (segment (start 40 6) (end 52 6) (width 1.0) (layer "F.Cu") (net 5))
 (segment (start 40 8) (end 40 11) (width 1.0) (layer "F.Cu") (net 5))
 (segment (start 40 11) (end 48 11) (width 1.0) (layer "F.Cu") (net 5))
 (segment (start 48 11) (end 48 17.5) (width 1.0) (layer "F.Cu") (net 5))
 (segment (start 48 17.5) (end 43.04 17.5) (width 1.0) (layer "F.Cu") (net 5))
 (segment (start 40 11) (end 9.5 11) (width 1.0) (layer "F.Cu") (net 5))
 (segment (start 9.5 11) (end 9.5 34.5) (width 1.0) (layer "F.Cu") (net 5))
 (segment (start 9.5 15.0) (end 11.96 15.0) (width 1.0) (layer "F.Cu") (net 5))
 (segment (start 9.5 34.5) (end 37.96 34.5) (width 0.6) (layer "F.Cu") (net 5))
 (segment (start 37.96 34.5) (end 37.96 36) (width 0.6) (layer "F.Cu") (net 5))
 (segment (start 17.04 15.0) (end 37.96 15.0) (width 0.3) (layer "F.Cu") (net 11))
 (segment (start 17.04 17.5) (end 37.96 17.5) (width 0.3) (layer "F.Cu") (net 12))
 (segment (start 17.04 20.0) (end 37.96 20.0) (width 0.3) (layer "F.Cu") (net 13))
 (segment (start 17.04 22.5) (end 37.96 22.5) (width 0.3) (layer "F.Cu") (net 14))
 (segment (start 17.04 25.0) (end 37.96 25.0) (width 0.3) (layer "F.Cu") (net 15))
 (segment (start 17.04 27.5) (end 37.96 27.5) (width 0.3) (layer "F.Cu") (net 16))
 (segment (start 17.04 30.0) (end 37.96 30.0) (width 0.3) (layer "F.Cu") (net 17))
 (segment (start 43.04 20.0) (end 57 20.0) (width 0.5) (layer "F.Cu") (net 18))
 (segment (start 43.04 22.5) (end 57 22.5) (width 0.5) (layer "F.Cu") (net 19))
 (segment (start 43.04 25.0) (end 57 25.0) (width 0.5) (layer "F.Cu") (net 20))
 (segment (start 43.04 27.5) (end 57 27.5) (width 0.5) (layer "F.Cu") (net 21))
 (segment (start 11.96 20.0) (end 8 20.0) (width 0.3) (layer "B.Cu") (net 6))
 (segment (start 8 20.0) (end 8 21.494999999999997) (width 0.3) (layer "B.Cu") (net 6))
 (segment (start 8 21.494999999999997) (end 6 21.494999999999997) (width 0.3) (layer "B.Cu") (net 6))
 (segment (start 11.96 22.5) (end 10 22.5) (width 0.3) (layer "B.Cu") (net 7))
 (segment (start 10 22.5) (end 10 24.035) (width 0.3) (layer "B.Cu") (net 7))
 (segment (start 10 24.035) (end 6 24.035) (width 0.3) (layer "B.Cu") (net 7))
 (segment (start 11.96 25.0) (end 11 25.0) (width 0.3) (layer "B.Cu") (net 8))
 (segment (start 11 25.0) (end 11 25.305) (width 0.3) (layer "B.Cu") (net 8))
 (segment (start 11 25.305) (end 6 25.305) (width 0.3) (layer "B.Cu") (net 8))
 (segment (start 27.04 36) (end 29 36) (width 0.3) (layer "F.Cu") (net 22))
 (segment (start 43.04 36) (end 45 36) (width 0.3) (layer "F.Cu") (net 23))
 (segment (start 37.46 8) (end 37.46 5.2) (width 0.5) (layer "B.Cu") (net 2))
 (segment (start 37.46 5.2) (end 42.54 5.2) (width 0.5) (layer "B.Cu") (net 2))
 (segment (start 42.54 5.2) (end 42.54 8) (width 0.5) (layer "B.Cu") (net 2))
 (segment (start 42.54 8) (end 49 8) (width 0.5) (layer "B.Cu") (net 2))
 (segment (start 49 8) (end 49 37.5) (width 0.5) (layer "B.Cu") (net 2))
 (segment (start 49 13) (end 52 13) (width 0.5) (layer "B.Cu") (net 2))
 (segment (start 52 13) (end 52 10) (width 0.5) (layer "B.Cu") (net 2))
 (segment (start 9 37.5) (end 49 37.5) (width 0.5) (layer "B.Cu") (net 2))
 (segment (start 33 36) (end 33 37.5) (width 0.5) (layer "B.Cu") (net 2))
 (segment (start 37.96 32.5) (end 35.5 32.5) (width 0.5) (layer "B.Cu") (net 2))
 (segment (start 35.5 32.5) (end 35.5 37.5) (width 0.5) (layer "B.Cu") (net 2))
 (segment (start 7 9) (end 7 17.5) (width 0.5) (layer "B.Cu") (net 2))
 (segment (start 11.96 17.5) (end 4.5 17.5) (width 0.5) (layer "B.Cu") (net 2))
 (segment (start 4.5 17.5) (end 4.5 33) (width 0.5) (layer "B.Cu") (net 2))
 (segment (start 4.5 22.765) (end 6 22.765) (width 0.5) (layer "B.Cu") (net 2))
 (segment (start 4.5 33) (end 9 33) (width 0.5) (layer "B.Cu") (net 2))
 (segment (start 9 33) (end 9 37.5) (width 0.5) (layer "B.Cu") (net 2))
 (gr_line (start 0 0) (end 60 0) (layer "Edge.Cuts") (width 0.05))
 (gr_line (start 60 0) (end 60 40) (layer "Edge.Cuts") (width 0.05))
 (gr_line (start 60 40) (end 0 40) (layer "Edge.Cuts") (width 0.05))
 (gr_line (start 0 40) (end 0 0) (layer "Edge.Cuts") (width 0.05)))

